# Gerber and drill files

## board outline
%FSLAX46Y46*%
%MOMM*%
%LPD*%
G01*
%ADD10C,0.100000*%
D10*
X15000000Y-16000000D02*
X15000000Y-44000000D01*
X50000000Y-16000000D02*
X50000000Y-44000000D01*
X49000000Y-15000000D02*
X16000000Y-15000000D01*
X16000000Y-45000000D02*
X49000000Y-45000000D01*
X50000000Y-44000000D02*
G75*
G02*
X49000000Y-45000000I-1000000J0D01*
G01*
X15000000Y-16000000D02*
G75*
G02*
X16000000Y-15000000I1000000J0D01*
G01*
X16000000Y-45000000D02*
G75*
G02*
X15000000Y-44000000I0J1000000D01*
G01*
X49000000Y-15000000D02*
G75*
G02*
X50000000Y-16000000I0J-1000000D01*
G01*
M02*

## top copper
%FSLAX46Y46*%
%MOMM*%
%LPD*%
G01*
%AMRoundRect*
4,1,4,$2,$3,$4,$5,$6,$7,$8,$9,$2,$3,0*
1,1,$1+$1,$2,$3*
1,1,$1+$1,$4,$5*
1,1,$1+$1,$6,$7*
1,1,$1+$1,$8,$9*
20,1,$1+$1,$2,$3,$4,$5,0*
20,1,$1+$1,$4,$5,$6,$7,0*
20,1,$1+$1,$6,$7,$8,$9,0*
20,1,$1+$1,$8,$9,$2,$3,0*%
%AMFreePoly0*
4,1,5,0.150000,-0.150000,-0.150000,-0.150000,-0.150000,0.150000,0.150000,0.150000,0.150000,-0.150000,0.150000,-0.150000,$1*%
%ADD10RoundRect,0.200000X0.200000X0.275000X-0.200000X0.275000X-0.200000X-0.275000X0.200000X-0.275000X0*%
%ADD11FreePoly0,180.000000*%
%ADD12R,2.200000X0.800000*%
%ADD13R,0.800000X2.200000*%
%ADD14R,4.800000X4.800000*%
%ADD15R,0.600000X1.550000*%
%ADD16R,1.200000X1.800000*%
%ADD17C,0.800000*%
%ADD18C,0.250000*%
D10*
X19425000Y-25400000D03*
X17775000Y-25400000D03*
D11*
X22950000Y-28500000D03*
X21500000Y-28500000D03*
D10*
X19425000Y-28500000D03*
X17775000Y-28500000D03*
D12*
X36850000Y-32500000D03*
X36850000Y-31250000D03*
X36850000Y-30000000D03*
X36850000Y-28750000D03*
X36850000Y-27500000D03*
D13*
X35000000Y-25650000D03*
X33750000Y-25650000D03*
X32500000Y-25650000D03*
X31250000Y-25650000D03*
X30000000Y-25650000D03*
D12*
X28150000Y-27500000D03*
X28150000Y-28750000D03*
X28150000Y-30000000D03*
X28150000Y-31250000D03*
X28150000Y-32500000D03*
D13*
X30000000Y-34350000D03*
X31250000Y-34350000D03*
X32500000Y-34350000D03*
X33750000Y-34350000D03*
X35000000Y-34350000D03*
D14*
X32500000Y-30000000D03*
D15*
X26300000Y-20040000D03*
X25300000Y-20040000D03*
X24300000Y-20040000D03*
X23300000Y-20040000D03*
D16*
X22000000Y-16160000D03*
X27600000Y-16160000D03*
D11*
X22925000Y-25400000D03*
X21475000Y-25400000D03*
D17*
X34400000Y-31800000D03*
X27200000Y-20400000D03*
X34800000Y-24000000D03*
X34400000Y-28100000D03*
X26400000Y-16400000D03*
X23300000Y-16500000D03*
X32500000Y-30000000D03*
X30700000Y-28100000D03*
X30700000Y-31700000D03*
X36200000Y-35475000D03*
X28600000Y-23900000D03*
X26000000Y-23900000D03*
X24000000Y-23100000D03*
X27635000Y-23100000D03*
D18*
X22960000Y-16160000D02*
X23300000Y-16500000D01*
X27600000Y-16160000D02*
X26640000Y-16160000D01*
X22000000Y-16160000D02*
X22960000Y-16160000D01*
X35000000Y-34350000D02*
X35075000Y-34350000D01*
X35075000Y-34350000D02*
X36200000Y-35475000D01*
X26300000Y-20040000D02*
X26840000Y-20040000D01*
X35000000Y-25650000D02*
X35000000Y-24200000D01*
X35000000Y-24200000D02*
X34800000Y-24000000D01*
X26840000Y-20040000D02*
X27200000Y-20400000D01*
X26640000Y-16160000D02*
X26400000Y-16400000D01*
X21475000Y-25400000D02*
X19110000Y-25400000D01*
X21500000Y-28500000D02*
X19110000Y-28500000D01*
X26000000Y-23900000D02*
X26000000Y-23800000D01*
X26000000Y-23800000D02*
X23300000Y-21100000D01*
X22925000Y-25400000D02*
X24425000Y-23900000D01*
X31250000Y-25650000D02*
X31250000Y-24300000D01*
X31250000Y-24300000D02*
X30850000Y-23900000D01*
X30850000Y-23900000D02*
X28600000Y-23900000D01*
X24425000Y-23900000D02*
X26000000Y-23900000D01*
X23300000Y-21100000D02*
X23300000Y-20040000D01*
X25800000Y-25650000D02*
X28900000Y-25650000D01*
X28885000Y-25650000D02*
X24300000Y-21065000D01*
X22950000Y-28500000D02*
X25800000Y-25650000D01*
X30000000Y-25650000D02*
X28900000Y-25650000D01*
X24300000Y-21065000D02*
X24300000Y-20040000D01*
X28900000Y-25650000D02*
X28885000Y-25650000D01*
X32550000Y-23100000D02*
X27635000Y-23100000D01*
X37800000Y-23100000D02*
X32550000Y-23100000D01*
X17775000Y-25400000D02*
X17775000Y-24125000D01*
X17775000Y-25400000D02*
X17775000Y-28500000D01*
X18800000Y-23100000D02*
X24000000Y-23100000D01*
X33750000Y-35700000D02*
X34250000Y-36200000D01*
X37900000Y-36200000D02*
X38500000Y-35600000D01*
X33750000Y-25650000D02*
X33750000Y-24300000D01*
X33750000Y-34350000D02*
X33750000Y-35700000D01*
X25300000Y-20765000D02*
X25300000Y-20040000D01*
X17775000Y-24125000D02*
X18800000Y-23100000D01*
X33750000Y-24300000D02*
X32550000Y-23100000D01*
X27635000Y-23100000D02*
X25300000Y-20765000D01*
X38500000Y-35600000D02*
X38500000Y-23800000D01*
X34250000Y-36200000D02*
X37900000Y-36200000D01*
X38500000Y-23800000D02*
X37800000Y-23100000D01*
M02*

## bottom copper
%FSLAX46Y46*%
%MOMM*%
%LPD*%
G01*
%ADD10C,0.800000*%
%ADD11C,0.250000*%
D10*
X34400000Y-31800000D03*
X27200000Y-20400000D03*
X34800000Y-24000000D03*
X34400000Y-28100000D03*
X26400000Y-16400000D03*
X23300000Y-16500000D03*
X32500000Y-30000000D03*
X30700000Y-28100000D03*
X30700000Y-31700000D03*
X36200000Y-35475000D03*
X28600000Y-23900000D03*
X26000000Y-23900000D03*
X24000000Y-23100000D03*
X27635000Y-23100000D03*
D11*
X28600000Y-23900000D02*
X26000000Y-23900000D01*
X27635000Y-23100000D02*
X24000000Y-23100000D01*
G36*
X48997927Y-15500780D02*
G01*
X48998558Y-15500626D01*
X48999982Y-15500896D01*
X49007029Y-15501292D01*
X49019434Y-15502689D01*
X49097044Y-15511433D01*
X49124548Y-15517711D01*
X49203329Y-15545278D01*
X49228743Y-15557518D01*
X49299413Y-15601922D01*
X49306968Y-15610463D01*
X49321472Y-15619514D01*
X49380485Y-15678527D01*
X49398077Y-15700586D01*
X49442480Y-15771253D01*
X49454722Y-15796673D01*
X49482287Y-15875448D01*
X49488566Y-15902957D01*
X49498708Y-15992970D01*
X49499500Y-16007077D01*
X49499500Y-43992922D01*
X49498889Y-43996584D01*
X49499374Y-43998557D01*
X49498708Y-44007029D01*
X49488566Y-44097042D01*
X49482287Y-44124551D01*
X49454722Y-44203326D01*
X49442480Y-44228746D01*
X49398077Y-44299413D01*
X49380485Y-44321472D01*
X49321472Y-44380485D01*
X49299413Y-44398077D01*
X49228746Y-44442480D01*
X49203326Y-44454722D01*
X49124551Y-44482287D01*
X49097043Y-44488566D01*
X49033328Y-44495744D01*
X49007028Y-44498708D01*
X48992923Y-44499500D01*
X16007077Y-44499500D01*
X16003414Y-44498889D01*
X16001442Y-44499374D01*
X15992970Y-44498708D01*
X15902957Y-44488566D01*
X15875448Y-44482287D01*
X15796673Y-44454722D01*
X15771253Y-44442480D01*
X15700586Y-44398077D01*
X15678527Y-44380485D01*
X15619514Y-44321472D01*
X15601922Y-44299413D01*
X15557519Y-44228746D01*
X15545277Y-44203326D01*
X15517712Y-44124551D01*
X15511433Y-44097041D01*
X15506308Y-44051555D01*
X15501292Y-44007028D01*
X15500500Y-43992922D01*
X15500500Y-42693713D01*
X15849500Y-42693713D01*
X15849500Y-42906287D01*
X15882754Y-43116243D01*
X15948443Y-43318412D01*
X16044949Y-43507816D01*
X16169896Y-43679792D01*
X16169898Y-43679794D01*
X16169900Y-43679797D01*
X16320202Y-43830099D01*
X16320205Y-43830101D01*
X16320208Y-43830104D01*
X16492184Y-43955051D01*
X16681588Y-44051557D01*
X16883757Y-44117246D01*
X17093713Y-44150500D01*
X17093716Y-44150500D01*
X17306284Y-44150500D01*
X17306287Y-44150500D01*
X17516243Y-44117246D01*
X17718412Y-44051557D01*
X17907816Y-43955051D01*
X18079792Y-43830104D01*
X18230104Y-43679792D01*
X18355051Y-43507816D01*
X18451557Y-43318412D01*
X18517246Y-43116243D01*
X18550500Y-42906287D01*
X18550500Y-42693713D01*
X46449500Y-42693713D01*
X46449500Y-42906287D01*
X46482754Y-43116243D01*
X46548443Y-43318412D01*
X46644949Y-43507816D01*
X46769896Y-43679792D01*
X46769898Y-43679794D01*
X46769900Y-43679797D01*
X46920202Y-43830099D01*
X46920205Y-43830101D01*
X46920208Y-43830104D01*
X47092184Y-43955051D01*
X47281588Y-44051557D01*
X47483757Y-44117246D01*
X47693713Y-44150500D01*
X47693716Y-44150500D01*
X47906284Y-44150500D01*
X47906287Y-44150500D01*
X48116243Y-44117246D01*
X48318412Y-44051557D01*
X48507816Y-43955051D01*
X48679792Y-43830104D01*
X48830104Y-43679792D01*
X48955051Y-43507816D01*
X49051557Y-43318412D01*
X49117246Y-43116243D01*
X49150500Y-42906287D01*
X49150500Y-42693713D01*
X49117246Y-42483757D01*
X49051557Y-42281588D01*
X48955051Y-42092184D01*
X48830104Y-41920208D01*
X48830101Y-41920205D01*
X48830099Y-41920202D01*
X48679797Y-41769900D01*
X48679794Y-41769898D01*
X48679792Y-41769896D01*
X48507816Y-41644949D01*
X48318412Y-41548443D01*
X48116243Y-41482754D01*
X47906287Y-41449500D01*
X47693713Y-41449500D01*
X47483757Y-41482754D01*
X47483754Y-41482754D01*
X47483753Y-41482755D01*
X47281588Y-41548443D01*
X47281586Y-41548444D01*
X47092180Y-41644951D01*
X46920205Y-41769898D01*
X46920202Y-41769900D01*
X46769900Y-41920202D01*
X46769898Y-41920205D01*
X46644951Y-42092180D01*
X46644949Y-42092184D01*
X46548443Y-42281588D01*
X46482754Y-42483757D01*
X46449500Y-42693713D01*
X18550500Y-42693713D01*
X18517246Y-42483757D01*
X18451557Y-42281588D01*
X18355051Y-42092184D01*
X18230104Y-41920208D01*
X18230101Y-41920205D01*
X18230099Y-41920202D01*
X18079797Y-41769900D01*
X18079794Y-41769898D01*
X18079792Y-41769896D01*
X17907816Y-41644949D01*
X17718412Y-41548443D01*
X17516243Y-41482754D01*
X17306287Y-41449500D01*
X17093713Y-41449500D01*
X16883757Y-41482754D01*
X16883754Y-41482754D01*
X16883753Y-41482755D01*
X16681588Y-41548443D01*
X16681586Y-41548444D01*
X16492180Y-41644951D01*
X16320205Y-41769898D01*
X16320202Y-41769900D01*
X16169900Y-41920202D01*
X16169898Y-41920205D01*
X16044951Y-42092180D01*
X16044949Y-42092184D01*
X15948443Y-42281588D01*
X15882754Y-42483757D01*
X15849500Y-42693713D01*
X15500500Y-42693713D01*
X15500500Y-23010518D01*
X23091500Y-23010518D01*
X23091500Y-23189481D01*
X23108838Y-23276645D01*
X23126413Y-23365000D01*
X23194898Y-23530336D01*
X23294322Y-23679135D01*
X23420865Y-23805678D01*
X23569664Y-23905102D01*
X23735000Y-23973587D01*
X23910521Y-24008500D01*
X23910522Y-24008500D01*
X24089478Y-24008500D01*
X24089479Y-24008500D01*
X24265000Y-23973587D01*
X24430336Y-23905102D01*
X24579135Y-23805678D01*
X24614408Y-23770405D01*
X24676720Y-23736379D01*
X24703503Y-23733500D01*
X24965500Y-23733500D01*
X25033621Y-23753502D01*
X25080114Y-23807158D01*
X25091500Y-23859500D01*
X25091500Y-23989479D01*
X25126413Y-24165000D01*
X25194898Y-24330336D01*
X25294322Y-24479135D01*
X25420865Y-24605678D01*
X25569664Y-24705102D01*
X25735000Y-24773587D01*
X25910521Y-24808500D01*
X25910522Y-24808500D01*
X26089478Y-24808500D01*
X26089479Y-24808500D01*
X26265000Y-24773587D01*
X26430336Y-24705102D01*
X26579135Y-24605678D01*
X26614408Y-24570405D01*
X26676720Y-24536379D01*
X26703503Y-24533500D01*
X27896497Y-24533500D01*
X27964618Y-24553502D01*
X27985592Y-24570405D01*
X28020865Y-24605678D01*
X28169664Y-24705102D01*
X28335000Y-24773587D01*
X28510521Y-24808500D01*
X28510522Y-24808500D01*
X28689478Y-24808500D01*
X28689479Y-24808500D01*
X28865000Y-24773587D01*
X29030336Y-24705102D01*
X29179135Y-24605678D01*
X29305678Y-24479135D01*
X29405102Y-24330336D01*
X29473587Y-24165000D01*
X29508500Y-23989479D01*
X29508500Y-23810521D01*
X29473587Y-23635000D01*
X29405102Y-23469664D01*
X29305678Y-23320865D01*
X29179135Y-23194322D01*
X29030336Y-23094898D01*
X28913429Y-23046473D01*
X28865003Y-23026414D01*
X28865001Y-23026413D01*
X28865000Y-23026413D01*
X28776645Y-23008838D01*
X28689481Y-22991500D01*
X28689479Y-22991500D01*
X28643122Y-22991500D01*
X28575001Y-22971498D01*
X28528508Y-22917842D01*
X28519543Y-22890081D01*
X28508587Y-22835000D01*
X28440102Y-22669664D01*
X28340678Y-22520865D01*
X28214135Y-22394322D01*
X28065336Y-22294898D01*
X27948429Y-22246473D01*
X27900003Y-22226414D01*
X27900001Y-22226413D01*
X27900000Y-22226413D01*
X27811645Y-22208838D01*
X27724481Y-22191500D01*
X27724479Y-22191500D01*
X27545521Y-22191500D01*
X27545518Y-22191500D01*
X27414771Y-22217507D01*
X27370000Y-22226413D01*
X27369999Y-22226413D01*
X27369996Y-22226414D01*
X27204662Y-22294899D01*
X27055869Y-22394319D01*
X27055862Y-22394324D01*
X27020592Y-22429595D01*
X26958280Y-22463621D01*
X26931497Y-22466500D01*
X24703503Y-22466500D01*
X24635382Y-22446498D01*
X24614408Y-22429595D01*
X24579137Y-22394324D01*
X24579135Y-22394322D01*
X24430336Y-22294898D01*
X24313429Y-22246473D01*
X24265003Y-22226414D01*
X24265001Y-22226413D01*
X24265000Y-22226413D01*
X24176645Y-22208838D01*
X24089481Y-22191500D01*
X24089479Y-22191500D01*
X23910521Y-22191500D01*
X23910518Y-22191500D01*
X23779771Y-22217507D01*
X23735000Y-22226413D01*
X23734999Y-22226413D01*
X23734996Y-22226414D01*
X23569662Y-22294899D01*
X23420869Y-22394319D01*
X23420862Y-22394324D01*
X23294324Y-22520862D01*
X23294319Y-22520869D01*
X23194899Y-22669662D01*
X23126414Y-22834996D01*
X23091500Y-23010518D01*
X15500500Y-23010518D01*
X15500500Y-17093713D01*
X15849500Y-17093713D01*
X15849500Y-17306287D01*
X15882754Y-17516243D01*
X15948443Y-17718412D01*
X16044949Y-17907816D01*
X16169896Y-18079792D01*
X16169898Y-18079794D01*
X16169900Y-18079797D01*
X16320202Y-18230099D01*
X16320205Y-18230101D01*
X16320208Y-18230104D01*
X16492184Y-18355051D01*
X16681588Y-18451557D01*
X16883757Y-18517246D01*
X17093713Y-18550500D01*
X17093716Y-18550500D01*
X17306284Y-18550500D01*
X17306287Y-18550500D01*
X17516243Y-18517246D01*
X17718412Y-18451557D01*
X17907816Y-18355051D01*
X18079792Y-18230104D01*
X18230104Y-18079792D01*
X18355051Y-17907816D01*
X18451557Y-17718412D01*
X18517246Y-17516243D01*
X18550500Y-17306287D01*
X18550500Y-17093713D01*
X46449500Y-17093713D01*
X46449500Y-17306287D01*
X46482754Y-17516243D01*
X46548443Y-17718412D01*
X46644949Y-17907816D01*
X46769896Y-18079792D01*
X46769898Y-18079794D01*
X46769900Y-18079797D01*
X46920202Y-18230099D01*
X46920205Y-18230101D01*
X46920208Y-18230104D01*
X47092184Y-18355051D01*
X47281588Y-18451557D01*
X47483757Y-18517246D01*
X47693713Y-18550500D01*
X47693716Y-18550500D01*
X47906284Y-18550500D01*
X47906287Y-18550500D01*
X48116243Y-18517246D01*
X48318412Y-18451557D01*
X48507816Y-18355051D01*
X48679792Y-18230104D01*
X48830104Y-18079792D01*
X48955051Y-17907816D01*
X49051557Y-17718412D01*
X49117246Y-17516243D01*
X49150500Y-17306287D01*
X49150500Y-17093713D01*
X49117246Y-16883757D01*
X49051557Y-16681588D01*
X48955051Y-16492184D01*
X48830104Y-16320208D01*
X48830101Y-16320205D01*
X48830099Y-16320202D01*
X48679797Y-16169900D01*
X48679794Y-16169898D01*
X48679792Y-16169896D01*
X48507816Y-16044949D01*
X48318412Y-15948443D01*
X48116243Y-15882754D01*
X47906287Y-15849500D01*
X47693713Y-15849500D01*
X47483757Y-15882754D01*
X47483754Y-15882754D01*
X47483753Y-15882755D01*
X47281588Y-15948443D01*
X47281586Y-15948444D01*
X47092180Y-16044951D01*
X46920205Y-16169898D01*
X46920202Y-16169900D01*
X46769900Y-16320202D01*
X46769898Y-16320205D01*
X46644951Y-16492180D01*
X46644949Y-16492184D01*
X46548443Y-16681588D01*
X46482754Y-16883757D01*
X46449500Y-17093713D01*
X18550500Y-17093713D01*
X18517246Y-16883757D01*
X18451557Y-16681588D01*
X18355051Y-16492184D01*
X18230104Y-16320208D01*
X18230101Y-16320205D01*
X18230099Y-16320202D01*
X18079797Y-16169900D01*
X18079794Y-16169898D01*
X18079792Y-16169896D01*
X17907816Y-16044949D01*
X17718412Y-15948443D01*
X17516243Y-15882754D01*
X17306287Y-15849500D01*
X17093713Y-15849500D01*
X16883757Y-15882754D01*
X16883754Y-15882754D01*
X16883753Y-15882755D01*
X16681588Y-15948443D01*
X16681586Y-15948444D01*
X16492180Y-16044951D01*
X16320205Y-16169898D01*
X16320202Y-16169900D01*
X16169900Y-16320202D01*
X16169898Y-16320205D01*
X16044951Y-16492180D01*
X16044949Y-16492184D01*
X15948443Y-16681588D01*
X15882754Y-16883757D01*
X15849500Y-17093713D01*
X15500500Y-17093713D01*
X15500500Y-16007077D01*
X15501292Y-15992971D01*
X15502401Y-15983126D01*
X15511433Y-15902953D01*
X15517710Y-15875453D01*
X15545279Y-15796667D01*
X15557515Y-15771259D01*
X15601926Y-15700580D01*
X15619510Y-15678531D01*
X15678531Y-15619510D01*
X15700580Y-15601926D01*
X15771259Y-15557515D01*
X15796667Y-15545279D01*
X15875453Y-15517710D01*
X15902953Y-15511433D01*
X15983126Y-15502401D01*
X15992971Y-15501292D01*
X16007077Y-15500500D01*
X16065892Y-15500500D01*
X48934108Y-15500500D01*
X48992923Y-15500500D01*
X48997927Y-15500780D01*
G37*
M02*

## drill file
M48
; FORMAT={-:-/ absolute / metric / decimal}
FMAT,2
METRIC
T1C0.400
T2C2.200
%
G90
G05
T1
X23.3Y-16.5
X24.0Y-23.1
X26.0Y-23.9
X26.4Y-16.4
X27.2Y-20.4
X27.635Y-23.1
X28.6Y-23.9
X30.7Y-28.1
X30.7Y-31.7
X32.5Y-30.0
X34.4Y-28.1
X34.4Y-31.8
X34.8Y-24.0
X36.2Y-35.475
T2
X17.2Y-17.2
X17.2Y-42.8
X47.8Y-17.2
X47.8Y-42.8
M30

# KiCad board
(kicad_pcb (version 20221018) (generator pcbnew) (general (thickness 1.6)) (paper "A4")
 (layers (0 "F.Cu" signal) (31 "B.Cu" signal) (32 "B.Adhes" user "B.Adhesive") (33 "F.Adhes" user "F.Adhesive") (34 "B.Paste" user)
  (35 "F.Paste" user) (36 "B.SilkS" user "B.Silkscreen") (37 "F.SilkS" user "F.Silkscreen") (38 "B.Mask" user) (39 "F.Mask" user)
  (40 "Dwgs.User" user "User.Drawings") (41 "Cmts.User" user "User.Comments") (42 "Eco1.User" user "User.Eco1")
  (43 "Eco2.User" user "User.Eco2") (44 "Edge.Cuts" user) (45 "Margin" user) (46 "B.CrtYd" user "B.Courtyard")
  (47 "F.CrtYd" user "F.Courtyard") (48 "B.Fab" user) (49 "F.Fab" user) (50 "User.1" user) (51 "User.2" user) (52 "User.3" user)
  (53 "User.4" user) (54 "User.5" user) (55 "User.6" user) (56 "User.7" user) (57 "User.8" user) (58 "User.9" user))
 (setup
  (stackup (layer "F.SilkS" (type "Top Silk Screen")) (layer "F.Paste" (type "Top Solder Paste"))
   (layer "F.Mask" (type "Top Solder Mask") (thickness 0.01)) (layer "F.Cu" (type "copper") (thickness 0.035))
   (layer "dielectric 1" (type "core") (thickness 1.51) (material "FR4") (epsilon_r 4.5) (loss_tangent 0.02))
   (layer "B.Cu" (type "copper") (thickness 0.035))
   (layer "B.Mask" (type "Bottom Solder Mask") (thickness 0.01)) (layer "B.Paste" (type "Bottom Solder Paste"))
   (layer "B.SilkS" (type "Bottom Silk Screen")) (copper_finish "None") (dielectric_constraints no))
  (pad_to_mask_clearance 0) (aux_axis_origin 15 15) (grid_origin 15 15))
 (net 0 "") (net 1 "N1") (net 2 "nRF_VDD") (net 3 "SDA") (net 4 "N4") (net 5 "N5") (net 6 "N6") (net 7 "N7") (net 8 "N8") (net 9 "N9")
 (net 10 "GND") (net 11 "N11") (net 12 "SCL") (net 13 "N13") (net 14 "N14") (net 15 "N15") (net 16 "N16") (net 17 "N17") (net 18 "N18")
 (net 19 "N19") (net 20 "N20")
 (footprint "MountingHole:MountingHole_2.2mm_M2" (layer "F.Cu") (at 17.2 17.2)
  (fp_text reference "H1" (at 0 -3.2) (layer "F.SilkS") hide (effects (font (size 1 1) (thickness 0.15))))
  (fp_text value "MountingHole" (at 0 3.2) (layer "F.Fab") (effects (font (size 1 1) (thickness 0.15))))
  (pad "" np_thru_hole circle (at 0 0) (size 2.2 2.2) (drill 2.2) (layers "*.Cu" "*.Mask")))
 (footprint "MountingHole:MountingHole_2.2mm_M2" (layer "F.Cu") (at 17.2 42.8)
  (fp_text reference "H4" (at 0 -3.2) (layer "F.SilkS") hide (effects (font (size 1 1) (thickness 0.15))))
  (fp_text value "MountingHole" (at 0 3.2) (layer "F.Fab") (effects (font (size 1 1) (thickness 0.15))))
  (pad "" np_thru_hole circle (at 0 0) (size 2.2 2.2) (drill 2.2) (layers "*.Cu" "*.Mask")))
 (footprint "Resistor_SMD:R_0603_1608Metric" (layer "F.Cu") (at 18.6 25.4 180)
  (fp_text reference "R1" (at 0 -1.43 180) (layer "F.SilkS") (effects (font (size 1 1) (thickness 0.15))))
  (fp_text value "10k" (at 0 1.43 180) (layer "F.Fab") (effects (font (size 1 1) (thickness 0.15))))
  (pad "1" smd roundrect (at -0.825 0 180) (size 0.8 0.95) (layers "F.Cu" "F.Paste" "F.Mask") (roundrect_rratio 0.25) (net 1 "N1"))
  (pad "2" smd roundrect (at 0.825 0 180) (size 0.8 0.95) (layers "F.Cu" "F.Paste" "F.Mask") (roundrect_rratio 0.25) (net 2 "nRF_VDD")))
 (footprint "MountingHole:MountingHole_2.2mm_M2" (layer "F.Cu") (at 47.8 17.2)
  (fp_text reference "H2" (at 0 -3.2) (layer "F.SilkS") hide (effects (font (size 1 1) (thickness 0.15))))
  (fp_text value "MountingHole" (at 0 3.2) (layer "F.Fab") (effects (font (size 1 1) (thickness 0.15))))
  (pad "" np_thru_hole circle (at 0 0) (size 2.2 2.2) (drill 2.2) (layers "*.Cu" "*.Mask")))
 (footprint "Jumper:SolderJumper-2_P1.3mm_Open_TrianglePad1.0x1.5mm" (layer "F.Cu") (at 22.225 28.5 180) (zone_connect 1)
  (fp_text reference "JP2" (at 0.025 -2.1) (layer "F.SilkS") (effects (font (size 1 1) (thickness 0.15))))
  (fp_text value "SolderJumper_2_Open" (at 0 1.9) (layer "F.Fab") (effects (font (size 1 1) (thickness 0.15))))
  (pad "1" smd custom (at -0.725 0 180) (size 0.3 0.3) (layers "F.Cu" "F.Mask") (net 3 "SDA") (zone_connect 2) (thermal_bridge_angle 45)
   (options (clearance outline) (anchor rect)) (primitives))
  (pad "2" smd custom (at 0.725 0 180) (size 0.3 0.3) (layers "F.Cu" "F.Mask") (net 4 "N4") (zone_connect 2) (thermal_bridge_angle 45)
   (options (clearance outline) (anchor rect)) (primitives)))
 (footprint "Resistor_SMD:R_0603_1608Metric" (layer "F.Cu") (at 18.6 28.5 180)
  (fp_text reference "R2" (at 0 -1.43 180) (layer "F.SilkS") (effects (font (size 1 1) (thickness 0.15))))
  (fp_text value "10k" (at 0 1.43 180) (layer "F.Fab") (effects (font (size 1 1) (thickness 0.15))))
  (pad "1" smd roundrect (at -0.825 0 180) (size 0.8 0.95) (layers "F.Cu" "F.Paste" "F.Mask") (roundrect_rratio 0.25) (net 4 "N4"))
  (pad "2" smd roundrect (at 0.825 0 180) (size 0.8 0.95) (layers "F.Cu" "F.Paste" "F.Mask") (roundrect_rratio 0.25) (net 2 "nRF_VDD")))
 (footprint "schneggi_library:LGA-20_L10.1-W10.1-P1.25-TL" (layer "F.Cu") (at 32.5 30 180)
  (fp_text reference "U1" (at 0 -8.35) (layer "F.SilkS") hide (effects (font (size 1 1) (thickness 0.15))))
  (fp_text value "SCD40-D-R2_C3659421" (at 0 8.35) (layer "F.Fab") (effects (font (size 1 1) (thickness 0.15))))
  (pad "1" smd rect (at -4.35 -2.5 180) (size 2.2 0.8) (layers "F.Cu" "F.Paste" "F.Mask") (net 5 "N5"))
  (pad "2" smd rect (at -4.35 -1.25 180) (size 2.2 0.8) (layers "F.Cu" "F.Paste" "F.Mask") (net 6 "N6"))
  (pad "3" smd rect (at -4.35 0 180) (size 2.2 0.8) (layers "F.Cu" "F.Paste" "F.Mask") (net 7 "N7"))
  (pad "4" smd rect (at -4.35 1.25 180) (size 2.2 0.8) (layers "F.Cu" "F.Paste" "F.Mask") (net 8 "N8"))
  (pad "5" smd rect (at -4.35 2.5 180) (size 2.2 0.8) (layers "F.Cu" "F.Paste" "F.Mask") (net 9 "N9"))
  (pad "6" smd rect (at -2.5 4.35 270) (size 2.2 0.8) (layers "F.Cu" "F.Paste" "F.Mask") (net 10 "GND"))
  (pad "7" smd rect (at -1.25 4.35 270) (size 2.2 0.8) (layers "F.Cu" "F.Paste" "F.Mask") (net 2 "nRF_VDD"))
  (pad "8" smd rect (at 0 4.35 270) (size 2.2 0.8) (layers "F.Cu" "F.Paste" "F.Mask") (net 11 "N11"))
  (pad "9" smd rect (at 1.25 4.35 270) (size 2.2 0.8) (layers "F.Cu" "F.Paste" "F.Mask") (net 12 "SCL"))
  (pad "10" smd rect (at 2.5 4.35 270) (size 2.2 0.8) (layers "F.Cu" "F.Paste" "F.Mask") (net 3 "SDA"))
  (pad "11" smd rect (at 4.35 2.5) (size 2.2 0.8) (layers "F.Cu" "F.Paste" "F.Mask") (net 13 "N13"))
  (pad "12" smd rect (at 4.35 1.25) (size 2.2 0.8) (layers "F.Cu" "F.Paste" "F.Mask") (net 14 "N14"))
  (pad "13" smd rect (at 4.35 0) (size 2.2 0.8) (layers "F.Cu" "F.Paste" "F.Mask") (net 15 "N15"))
  (pad "14" smd rect (at 4.35 -1.25) (size 2.2 0.8) (layers "F.Cu" "F.Paste" "F.Mask") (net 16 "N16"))
  (pad "15" smd rect (at 4.35 -2.5) (size 2.2 0.8) (layers "F.Cu" "F.Paste" "F.Mask") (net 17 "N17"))
  (pad "16" smd rect (at 2.5 -4.35 90) (size 2.2 0.8) (layers "F.Cu" "F.Paste" "F.Mask") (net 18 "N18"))
  (pad "17" smd rect (at 1.25 -4.35 90) (size 2.2 0.8) (layers "F.Cu" "F.Paste" "F.Mask") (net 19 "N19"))
  (pad "18" smd rect (at 0 -4.35 90) (size 2.2 0.8) (layers "F.Cu" "F.Paste" "F.Mask") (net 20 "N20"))
  (pad "19" smd rect (at -1.25 -4.35 90) (size 2.2 0.8) (layers "F.Cu" "F.Paste" "F.Mask") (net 2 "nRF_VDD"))
  (pad "20" smd rect (at -2.5 -4.35 90) (size 2.2 0.8) (layers "F.Cu" "F.Paste" "F.Mask") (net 10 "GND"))
  (pad "21" smd rect (at 0 0 90) (size 4.8 4.8) (layers "F.Cu" "F.Paste" "F.Mask") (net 10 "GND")))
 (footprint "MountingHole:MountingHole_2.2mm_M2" (layer "F.Cu") (at 47.8 42.8)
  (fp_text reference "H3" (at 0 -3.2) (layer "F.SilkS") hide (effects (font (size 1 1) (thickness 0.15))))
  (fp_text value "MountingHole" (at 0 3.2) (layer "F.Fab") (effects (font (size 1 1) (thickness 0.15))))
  (pad "" np_thru_hole circle (at 0 0) (size 2.2 2.2) (drill 2.2) (layers "*.Cu" "*.Mask")))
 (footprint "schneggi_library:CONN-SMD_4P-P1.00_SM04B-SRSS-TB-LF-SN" (layer "F.Cu") (at 24.8 18.1 180)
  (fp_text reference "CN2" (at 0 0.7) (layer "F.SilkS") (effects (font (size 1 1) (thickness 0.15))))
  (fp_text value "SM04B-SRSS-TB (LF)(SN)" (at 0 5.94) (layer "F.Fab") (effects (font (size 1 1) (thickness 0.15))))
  (pad "1" smd rect (at -1.5 -1.94 180) (size 0.6 1.55) (layers "F.Cu" "F.Paste" "F.Mask") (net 10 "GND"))
  (pad "2" smd rect (at -0.5 -1.94 180) (size 0.6 1.55) (layers "F.Cu" "F.Paste" "F.Mask") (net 2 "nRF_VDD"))
  (pad "3" smd rect (at 0.5 -1.94 180) (size 0.6 1.55) (layers "F.Cu" "F.Paste" "F.Mask") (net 3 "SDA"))
  (pad "4" smd rect (at 1.5 -1.94 180) (size 0.6 1.55) (layers "F.Cu" "F.Paste" "F.Mask") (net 12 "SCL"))
  (pad "5" smd rect (at 2.8 1.94 180) (size 1.2 1.8) (layers "F.Cu" "F.Paste" "F.Mask") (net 10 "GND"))
  (pad "6" smd rect (at -2.8 1.94 180) (size 1.2 1.8) (layers "F.Cu" "F.Paste" "F.Mask") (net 10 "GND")))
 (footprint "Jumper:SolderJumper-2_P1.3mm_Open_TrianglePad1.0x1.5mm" (layer "F.Cu") (at 22.2 25.4 180) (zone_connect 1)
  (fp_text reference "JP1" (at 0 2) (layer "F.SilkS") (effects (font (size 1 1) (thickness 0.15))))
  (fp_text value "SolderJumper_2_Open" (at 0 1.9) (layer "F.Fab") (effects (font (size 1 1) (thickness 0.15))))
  (pad "1" smd custom (at -0.725 0 180) (size 0.3 0.3) (layers "F.Cu" "F.Mask") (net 12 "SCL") (zone_connect 2) (thermal_bridge_angle 45)
   (options (clearance outline) (anchor rect)) (primitives))
  (pad "2" smd custom (at 0.725 0 180) (size 0.3 0.3) (layers "F.Cu" "F.Mask") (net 1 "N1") (zone_connect 2) (thermal_bridge_angle 45)
   (options (clearance outline) (anchor rect)) (primitives)))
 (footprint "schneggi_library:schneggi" (layer "F.Cu") (at 41.2 40.2)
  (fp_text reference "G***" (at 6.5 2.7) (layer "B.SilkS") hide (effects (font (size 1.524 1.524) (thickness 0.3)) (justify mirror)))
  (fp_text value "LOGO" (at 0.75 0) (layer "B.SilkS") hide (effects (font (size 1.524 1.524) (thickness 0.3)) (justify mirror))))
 (gr_line (start 15 16) (end 15 44) (stroke (width 0.1) (type solid)) (layer "Edge.Cuts"))
 (gr_line (start 50 16) (end 50 44) (stroke (width 0.1) (type solid)) (layer "Edge.Cuts"))
 (gr_line (start 49 15) (end 16 15) (stroke (width 0.1) (type solid)) (layer "Edge.Cuts"))
 (gr_line (start 16 45) (end 49 45) (stroke (width 0.1) (type solid)) (layer "Edge.Cuts"))
 (gr_arc (start 50 44) (mid 49.707107 44.707107) (end 49 45) (stroke (width 0.1) (type solid)) (layer "Edge.Cuts"))
 (gr_arc (start 15 16) (mid 15.292893 15.292893) (end 16 15) (stroke (width 0.1) (type solid)) (layer "Edge.Cuts"))
 (gr_arc (start 16 45) (mid 15.292893 44.707107) (end 15 44) (stroke (width 0.1) (type solid)) (layer "Edge.Cuts"))
 (gr_arc (start 49 15) (mid 49.707107 15.292893) (end 50 16) (stroke (width 0.1) (type solid)) (layer "Edge.Cuts"))
 (segment (start 22.96 16.16) (end 23.3 16.5) (width 0.25) (layer "F.Cu") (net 10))
 (segment (start 27.6 16.16) (end 26.64 16.16) (width 0.25) (layer "F.Cu") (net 10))
 (segment (start 22 16.16) (end 22.96 16.16) (width 0.25) (layer "F.Cu") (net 10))
 (segment (start 35 34.35) (end 35.075 34.35) (width 0.25) (layer "F.Cu") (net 10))
 (segment (start 35.075 34.35) (end 36.2 35.475) (width 0.25) (layer "F.Cu") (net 10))
 (segment (start 26.3 20.04) (end 26.84 20.04) (width 0.25) (layer "F.Cu") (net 10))
 (segment (start 35 25.65) (end 35 24.2) (width 0.25) (layer "F.Cu") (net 10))
 (segment (start 35 24.2) (end 34.8 24) (width 0.25) (layer "F.Cu") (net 10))
 (segment (start 26.84 20.04) (end 27.2 20.4) (width 0.25) (layer "F.Cu") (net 10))
 (segment (start 26.64 16.16) (end 26.4 16.4) (width 0.25) (layer "F.Cu") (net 10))
 (via (at 34.4 31.8) (size 0.8) (drill 0.4) (layers "F.Cu" "B.Cu") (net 10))
 (via (at 27.2 20.4) (size 0.8) (drill 0.4) (layers "F.Cu" "B.Cu") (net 10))
 (via (at 34.8 24) (size 0.8) (drill 0.4) (layers "F.Cu" "B.Cu") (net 10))
 (via (at 34.4 28.1) (size 0.8) (drill 0.4) (layers "F.Cu" "B.Cu") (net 10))
 (via (at 26.4 16.4) (size 0.8) (drill 0.4) (layers "F.Cu" "B.Cu") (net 10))
 (via (at 23.3 16.5) (size 0.8) (drill 0.4) (layers "F.Cu" "B.Cu") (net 10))
 (via (at 32.5 30) (size 0.8) (drill 0.4) (layers "F.Cu" "B.Cu") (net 10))
 (via (at 30.7 28.1) (size 0.8) (drill 0.4) (layers "F.Cu" "B.Cu") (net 10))
 (via (at 30.7 31.7) (size 0.8) (drill 0.4) (layers "F.Cu" "B.Cu") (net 10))
 (via (at 36.2 35.475) (size 0.8) (drill 0.4) (layers "F.Cu" "B.Cu") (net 10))
 (segment (start 21.475 25.4) (end 19.11 25.4) (width 0.25) (layer "F.Cu") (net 1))
 (segment (start 21.5 28.5) (end 19.11 28.5) (width 0.25) (layer "F.Cu") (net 4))
 (segment (start 26 23.9) (end 26 23.8) (width 0.25) (layer "F.Cu") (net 12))
 (segment (start 26 23.8) (end 23.3 21.1) (width 0.25) (layer "F.Cu") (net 12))
 (segment (start 22.925 25.4) (end 24.425 23.9) (width 0.25) (layer "F.Cu") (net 12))
 (segment (start 31.25 25.65) (end 31.25 24.3) (width 0.25) (layer "F.Cu") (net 12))
 (segment (start 31.25 24.3) (end 30.85 23.9) (width 0.25) (layer "F.Cu") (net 12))
 (segment (start 30.85 23.9) (end 28.6 23.9) (width 0.25) (layer "F.Cu") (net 12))
 (segment (start 24.425 23.9) (end 26 23.9) (width 0.25) (layer "F.Cu") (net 12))
 (segment (start 23.3 21.1) (end 23.3 20.04) (width 0.25) (layer "F.Cu") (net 12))
 (via (at 28.6 23.9) (size 0.8) (drill 0.4) (layers "F.Cu" "B.Cu") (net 12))
 (via (at 26 23.9) (size 0.8) (drill 0.4) (layers "F.Cu" "B.Cu") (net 12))
 (segment (start 28.6 23.9) (end 26 23.9) (width 0.25) (layer "B.Cu") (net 12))
 (segment (start 25.8 25.65) (end 28.9 25.65) (width 0.25) (layer "F.Cu") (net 3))
 (segment (start 28.885 25.65) (end 24.3 21.065) (width 0.25) (layer "F.Cu") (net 3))
 (segment (start 22.95 28.5) (end 25.8 25.65) (width 0.25) (layer "F.Cu") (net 3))
 (segment (start 30 25.65) (end 28.9 25.65) (width 0.25) (layer "F.Cu") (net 3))
 (segment (start 24.3 21.065) (end 24.3 20.04) (width 0.25) (layer "F.Cu") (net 3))
 (segment (start 28.9 25.65) (end 28.885 25.65) (width 0.25) (layer "F.Cu") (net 3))
 (segment (start 32.55 23.1) (end 27.635 23.1) (width 0.25) (layer "F.Cu") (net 2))
 (segment (start 37.8 23.1) (end 32.55 23.1) (width 0.25) (layer "F.Cu") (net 2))
 (segment (start 17.775 25.4) (end 17.775 24.125) (width 0.25) (layer "F.Cu") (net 2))
 (segment (start 17.775 25.4) (end 17.775 28.5) (width 0.25) (layer "F.Cu") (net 2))
 (segment (start 18.8 23.1) (end 24 23.1) (width 0.25) (layer "F.Cu") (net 2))
 (segment (start 33.75 35.7) (end 34.25 36.2) (width 0.25) (layer "F.Cu") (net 2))
 (segment (start 37.9 36.2) (end 38.5 35.6) (width 0.25) (layer "F.Cu") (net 2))
 (segment (start 33.75 25.65) (end 33.75 24.3) (width 0.25) (layer "F.Cu") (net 2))
 (segment (start 33.75 34.35) (end 33.75 35.7) (width 0.25) (layer "F.Cu") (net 2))
 (segment (start 25.3 20.765) (end 25.3 20.04) (width 0.25) (layer "F.Cu") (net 2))
 (segment (start 17.775 24.125) (end 18.8 23.1) (width 0.25) (layer "F.Cu") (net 2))
 (segment (start 33.75 24.3) (end 32.55 23.1) (width 0.25) (layer "F.Cu") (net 2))
 (segment (start 27.635 23.1) (end 25.3 20.765) (width 0.25) (layer "F.Cu") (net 2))
 (segment (start 38.5 35.6) (end 38.5 23.8) (width 0.25) (layer "F.Cu") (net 2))
 (segment (start 34.25 36.2) (end 37.9 36.2) (width 0.25) (layer "F.Cu") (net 2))
 (segment (start 38.5 23.8) (end 37.8 23.1) (width 0.25) (layer "F.Cu") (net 2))
 (via (at 24 23.1) (size 0.8) (drill 0.4) (layers "F.Cu" "B.Cu") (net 2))
 (via (at 27.635 23.1) (size 0.8) (drill 0.4) (layers "F.Cu" "B.Cu") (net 2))
 (segment (start 27.635 23.1) (end 24 23.1) (width 0.25) (layer "B.Cu") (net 2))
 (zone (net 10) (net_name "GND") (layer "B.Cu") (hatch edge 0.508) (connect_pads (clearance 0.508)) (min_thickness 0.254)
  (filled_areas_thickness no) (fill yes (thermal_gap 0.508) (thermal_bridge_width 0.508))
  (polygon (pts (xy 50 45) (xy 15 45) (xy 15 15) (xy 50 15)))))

